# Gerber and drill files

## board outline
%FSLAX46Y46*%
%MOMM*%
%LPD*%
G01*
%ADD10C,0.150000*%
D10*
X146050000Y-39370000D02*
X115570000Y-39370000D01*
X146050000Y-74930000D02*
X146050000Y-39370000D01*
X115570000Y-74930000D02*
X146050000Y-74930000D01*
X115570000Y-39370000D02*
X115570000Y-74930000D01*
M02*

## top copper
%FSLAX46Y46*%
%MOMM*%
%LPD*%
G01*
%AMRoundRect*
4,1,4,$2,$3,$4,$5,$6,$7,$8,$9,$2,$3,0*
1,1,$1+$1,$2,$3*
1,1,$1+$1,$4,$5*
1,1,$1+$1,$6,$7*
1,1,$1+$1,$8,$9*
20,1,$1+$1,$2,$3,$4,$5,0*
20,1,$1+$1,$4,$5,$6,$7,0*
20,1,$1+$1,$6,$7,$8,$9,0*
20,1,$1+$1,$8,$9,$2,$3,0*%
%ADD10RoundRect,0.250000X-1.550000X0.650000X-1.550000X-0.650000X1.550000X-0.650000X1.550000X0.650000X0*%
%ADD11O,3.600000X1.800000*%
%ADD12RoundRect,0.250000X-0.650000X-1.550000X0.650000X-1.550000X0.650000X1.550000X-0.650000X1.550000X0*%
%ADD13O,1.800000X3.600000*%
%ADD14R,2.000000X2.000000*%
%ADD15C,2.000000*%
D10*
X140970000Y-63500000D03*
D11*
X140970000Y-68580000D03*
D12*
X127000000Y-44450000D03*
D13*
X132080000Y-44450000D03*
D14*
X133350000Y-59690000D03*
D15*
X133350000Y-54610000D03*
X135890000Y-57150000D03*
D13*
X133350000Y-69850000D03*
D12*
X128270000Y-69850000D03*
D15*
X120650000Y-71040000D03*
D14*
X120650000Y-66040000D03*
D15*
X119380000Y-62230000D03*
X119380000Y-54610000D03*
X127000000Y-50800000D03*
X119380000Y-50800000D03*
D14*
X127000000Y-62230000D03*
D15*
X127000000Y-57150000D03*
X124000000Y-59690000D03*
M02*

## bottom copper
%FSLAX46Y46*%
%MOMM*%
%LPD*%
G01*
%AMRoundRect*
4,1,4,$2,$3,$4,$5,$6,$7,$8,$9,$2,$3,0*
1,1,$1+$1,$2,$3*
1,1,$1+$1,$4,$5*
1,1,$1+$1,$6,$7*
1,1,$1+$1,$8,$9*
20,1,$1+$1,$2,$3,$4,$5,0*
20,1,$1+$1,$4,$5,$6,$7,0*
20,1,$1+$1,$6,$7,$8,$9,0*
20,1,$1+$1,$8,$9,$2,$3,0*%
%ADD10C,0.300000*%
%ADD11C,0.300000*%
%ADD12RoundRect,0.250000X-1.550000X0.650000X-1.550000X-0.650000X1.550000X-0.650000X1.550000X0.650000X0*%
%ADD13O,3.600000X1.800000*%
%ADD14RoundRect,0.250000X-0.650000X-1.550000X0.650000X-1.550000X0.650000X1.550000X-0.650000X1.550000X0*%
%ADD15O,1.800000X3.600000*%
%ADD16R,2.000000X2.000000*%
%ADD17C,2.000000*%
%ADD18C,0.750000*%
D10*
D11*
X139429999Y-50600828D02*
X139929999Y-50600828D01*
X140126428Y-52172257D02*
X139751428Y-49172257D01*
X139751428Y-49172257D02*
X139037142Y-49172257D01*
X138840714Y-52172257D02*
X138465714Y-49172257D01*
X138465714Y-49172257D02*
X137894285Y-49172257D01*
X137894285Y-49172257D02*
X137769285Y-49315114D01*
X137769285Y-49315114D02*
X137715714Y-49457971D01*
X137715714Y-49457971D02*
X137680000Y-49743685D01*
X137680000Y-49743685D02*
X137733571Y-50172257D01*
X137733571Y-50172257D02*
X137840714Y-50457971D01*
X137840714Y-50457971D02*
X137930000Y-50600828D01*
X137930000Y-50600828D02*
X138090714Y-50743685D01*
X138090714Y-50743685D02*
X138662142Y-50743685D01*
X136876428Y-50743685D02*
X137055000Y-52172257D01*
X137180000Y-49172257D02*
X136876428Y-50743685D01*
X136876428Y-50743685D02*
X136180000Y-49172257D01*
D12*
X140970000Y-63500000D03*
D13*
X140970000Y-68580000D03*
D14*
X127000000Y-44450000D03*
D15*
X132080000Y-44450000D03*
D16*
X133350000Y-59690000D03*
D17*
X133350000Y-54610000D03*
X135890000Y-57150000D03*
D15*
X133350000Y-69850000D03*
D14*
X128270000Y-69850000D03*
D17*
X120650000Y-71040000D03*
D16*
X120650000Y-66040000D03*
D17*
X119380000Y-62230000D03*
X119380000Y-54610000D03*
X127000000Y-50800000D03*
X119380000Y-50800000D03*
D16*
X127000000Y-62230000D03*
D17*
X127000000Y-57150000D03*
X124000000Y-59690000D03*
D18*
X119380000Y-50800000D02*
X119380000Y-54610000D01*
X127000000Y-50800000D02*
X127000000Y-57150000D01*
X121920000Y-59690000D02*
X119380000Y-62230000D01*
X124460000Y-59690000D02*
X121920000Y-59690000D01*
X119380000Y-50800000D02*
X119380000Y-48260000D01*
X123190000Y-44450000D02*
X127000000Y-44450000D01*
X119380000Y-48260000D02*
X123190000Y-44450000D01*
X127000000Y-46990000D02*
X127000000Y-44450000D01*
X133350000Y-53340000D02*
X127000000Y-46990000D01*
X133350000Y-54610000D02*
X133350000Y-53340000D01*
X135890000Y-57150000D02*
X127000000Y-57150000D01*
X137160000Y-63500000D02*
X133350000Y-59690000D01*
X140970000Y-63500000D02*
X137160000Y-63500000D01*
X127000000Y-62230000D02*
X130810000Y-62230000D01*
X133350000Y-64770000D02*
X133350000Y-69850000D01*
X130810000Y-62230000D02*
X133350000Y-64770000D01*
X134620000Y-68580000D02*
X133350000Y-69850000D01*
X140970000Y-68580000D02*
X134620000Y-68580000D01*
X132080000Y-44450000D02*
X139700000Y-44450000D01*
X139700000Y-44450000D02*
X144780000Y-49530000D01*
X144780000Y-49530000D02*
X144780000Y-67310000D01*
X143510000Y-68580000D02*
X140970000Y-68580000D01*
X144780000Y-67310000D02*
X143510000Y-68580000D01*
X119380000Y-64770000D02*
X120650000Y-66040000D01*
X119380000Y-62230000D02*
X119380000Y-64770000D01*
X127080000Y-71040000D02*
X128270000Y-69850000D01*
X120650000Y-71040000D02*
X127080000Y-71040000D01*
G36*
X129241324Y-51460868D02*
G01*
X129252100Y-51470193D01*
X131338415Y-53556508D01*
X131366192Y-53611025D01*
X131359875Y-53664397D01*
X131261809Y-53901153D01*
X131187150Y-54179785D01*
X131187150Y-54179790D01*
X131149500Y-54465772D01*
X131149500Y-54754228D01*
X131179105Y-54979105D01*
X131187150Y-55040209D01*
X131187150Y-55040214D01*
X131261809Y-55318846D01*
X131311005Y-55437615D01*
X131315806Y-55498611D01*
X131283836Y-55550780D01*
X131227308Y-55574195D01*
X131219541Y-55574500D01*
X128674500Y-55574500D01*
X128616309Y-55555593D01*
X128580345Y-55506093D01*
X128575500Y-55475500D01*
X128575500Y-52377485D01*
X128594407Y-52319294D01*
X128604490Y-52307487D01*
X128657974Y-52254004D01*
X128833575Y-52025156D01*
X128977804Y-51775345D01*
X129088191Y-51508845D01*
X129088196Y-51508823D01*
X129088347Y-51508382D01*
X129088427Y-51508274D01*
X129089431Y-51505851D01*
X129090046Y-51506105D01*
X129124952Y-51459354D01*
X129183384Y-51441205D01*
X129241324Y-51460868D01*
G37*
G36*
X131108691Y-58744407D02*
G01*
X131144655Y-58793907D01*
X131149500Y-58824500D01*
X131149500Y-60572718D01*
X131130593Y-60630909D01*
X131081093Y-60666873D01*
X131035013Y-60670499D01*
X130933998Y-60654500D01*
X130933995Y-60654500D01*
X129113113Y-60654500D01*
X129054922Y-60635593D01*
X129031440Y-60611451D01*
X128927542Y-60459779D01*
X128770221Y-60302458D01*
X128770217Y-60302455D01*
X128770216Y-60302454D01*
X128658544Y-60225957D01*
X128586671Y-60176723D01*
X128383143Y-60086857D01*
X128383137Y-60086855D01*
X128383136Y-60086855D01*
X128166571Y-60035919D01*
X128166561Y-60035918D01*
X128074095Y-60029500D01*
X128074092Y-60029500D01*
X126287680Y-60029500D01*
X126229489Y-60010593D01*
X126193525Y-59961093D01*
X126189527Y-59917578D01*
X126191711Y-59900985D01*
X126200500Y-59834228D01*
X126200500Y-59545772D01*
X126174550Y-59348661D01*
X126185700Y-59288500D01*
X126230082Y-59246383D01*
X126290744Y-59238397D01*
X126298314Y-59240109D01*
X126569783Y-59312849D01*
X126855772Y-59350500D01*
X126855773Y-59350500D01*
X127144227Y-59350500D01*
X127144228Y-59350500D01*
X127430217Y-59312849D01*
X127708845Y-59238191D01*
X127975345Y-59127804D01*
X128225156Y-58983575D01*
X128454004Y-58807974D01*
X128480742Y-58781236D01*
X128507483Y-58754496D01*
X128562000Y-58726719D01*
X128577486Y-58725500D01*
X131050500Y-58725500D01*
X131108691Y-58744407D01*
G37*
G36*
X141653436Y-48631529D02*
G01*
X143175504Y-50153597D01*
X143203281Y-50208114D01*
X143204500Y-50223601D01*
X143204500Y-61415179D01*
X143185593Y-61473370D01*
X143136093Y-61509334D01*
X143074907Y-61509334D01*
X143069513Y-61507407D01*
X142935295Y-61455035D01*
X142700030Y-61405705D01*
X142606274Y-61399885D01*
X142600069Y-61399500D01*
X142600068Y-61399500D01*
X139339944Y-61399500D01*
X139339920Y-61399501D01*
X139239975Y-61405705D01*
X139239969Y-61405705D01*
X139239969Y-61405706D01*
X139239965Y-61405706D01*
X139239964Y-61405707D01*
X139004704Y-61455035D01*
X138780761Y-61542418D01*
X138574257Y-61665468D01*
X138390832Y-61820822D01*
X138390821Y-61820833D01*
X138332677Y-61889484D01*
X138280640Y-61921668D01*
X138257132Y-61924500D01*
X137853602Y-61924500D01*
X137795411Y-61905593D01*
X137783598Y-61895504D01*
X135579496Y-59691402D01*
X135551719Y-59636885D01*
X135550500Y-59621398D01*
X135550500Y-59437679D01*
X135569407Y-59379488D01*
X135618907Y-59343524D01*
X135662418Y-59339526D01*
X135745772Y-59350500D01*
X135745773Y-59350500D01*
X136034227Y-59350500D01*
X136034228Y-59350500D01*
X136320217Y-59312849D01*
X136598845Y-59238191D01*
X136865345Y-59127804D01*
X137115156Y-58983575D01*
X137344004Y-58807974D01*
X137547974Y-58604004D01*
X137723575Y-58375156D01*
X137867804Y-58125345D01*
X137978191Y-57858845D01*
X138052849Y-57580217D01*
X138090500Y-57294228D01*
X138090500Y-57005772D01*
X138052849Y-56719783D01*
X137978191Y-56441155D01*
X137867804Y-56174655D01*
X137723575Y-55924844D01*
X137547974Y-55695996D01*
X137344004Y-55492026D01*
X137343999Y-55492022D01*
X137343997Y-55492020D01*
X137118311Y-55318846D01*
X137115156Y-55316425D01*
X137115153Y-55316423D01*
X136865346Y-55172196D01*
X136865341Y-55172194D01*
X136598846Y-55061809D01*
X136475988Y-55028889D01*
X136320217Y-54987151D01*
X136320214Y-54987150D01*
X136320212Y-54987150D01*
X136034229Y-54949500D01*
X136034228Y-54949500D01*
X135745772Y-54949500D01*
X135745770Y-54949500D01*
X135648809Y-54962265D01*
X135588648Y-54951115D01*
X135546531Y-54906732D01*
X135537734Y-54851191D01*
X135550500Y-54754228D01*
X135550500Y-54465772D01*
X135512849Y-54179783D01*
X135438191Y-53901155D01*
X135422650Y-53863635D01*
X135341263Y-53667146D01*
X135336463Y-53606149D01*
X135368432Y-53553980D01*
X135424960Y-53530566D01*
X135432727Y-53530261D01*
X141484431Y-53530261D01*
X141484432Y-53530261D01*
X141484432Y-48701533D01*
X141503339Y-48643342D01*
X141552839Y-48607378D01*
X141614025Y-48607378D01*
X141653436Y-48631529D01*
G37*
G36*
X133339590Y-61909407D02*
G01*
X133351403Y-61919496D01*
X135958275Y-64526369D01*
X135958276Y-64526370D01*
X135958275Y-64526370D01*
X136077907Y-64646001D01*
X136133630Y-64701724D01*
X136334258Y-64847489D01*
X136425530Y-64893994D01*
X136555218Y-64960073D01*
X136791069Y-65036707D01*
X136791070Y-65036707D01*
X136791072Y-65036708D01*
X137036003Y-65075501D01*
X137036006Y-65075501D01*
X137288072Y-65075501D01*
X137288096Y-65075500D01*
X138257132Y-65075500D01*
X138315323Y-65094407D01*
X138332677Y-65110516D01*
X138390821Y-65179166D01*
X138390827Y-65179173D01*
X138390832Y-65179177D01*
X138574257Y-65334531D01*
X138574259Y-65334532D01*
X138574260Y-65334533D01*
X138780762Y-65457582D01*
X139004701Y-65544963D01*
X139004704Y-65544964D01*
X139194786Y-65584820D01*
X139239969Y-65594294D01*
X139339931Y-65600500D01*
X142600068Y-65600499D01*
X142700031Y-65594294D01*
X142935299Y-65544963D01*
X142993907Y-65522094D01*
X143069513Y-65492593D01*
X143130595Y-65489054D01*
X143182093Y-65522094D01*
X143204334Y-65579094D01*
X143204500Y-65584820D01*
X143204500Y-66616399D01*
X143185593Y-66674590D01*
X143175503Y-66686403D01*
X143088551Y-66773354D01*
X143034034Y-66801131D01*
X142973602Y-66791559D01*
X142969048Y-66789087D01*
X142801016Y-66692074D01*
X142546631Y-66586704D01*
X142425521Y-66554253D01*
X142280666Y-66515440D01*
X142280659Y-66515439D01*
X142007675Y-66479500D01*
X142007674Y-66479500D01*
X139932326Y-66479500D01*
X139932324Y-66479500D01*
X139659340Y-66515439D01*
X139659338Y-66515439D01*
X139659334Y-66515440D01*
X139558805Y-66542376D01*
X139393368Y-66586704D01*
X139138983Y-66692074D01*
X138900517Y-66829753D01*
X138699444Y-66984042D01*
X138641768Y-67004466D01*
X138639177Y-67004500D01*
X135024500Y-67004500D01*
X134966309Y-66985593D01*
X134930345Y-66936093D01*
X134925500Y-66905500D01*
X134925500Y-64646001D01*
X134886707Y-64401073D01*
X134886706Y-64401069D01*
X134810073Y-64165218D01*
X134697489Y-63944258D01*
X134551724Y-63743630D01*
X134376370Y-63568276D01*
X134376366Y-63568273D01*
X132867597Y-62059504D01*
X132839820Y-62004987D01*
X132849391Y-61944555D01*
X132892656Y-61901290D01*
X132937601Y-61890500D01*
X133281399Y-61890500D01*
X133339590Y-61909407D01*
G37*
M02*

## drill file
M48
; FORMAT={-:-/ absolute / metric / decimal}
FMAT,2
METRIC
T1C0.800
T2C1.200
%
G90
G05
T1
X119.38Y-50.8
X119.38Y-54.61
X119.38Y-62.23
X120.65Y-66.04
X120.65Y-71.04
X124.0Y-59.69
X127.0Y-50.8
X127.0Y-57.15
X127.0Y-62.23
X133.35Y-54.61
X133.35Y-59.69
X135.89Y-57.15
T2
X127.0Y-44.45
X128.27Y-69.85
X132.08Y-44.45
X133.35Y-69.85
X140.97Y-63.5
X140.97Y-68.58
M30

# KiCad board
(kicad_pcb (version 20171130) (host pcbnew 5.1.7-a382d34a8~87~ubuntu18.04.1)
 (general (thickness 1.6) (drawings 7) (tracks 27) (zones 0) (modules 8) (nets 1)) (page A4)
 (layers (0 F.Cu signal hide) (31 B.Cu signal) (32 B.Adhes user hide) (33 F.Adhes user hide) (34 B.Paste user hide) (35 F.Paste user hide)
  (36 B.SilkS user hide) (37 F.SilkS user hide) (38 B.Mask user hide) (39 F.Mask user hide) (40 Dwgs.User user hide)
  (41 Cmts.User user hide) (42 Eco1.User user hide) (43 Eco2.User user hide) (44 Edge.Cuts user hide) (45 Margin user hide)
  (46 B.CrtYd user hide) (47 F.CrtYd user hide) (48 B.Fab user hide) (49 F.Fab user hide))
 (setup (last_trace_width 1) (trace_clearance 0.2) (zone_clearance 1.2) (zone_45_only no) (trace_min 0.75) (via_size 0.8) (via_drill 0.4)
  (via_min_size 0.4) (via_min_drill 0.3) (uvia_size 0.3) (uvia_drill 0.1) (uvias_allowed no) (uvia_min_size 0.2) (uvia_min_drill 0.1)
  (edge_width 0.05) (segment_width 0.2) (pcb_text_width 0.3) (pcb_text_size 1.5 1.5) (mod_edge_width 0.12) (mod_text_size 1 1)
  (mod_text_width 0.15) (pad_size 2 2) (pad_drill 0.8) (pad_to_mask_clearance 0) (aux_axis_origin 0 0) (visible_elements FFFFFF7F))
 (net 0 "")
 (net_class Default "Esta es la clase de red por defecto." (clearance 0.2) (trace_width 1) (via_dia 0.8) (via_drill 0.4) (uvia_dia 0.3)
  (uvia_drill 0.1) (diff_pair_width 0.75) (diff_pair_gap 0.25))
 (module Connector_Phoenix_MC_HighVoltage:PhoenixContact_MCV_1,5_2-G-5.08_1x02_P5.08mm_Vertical (layer F.Cu) (at 140.97 63.5 270)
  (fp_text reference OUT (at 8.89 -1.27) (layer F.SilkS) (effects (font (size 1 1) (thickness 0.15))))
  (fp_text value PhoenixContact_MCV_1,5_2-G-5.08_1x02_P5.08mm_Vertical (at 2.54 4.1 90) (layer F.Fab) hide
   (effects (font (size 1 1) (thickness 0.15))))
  (pad 1 thru_hole roundrect (at 0 0 270) (size 1.8 3.6) (drill 1.2) (layers *.Cu *.Mask) (roundrect_rratio 0.1388888888888889))
  (pad 2 thru_hole oval (at 5.08 0 270) (size 1.8 3.6) (drill 1.2) (layers *.Cu *.Mask)))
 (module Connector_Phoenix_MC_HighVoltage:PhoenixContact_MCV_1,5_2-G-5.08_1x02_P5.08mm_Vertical (layer F.Cu) (at 127 44.45)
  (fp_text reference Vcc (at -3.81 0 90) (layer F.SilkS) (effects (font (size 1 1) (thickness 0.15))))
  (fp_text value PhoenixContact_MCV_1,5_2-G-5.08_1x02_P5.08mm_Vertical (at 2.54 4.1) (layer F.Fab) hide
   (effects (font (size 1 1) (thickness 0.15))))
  (pad 1 thru_hole roundrect (at 0 0) (size 1.8 3.6) (drill 1.2) (layers *.Cu *.Mask) (roundrect_rratio 0.1388888888888889))
  (pad 2 thru_hole oval (at 5.08 0) (size 1.8 3.6) (drill 1.2) (layers *.Cu *.Mask)))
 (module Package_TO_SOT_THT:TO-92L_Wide (layer B.Cu) (at 133.35 59.69 90)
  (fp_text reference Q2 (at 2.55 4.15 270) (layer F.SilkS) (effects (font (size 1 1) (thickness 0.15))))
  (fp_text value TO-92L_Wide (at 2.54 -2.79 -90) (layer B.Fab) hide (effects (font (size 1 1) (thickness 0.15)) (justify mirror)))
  (pad 1 thru_hole rect (at 0 0 90) (size 2 2) (drill 0.8) (layers *.Cu *.Mask))
  (pad 3 thru_hole circle (at 5.08 0 90) (size 2 2) (drill 0.8) (layers *.Cu *.Mask))
  (pad 2 thru_hole circle (at 2.54 2.54 90) (size 2 2) (drill 0.8) (layers *.Cu *.Mask)))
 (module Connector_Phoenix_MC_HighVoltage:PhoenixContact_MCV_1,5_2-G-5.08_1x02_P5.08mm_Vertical (layer B.Cu) (at 128.27 69.85)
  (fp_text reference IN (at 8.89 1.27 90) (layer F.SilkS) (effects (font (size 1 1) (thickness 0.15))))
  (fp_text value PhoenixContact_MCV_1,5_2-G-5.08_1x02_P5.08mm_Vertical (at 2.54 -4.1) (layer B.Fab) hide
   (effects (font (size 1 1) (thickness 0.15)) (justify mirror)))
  (pad 2 thru_hole oval (at 5.08 0) (size 1.8 3.6) (drill 1.2) (layers *.Cu *.Mask))
  (pad 1 thru_hole roundrect (at 0 0) (size 1.8 3.6) (drill 1.2) (layers *.Cu *.Mask) (roundrect_rratio 0.1388888888888889)))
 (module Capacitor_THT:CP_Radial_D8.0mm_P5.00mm (layer F.Cu) (at 120.65 66.04 270)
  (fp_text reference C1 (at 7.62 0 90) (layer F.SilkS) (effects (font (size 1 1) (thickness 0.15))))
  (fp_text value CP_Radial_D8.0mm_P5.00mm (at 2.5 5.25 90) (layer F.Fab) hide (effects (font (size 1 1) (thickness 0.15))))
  (pad 2 thru_hole circle (at 5 0 270) (size 2 2) (drill 0.8) (layers *.Cu *.Mask))
  (pad 1 thru_hole rect (at 0 0 270) (size 2 2) (drill 0.8) (layers *.Cu *.Mask)))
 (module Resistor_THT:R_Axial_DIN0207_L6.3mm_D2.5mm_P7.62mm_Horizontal (layer F.Cu) (at 119.38 62.23 90)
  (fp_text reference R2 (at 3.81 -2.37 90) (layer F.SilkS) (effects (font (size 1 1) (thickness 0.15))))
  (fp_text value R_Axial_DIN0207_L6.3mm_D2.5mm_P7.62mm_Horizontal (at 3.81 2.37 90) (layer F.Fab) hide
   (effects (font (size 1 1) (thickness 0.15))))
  (pad 1 thru_hole circle (at 0 0 90) (size 2 2) (drill 0.8) (layers *.Cu *.Mask))
  (pad 2 thru_hole circle (at 7.62 0 90) (size 2 2) (drill 0.8) (layers *.Cu *.Mask)))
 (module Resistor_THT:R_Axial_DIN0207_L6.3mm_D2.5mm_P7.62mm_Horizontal (layer F.Cu) (at 119.38 50.8)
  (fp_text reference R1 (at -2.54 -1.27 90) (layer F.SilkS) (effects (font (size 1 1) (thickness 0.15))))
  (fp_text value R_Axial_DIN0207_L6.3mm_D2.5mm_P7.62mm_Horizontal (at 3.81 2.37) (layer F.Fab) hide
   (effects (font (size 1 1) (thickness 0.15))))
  (pad 2 thru_hole circle (at 7.62 0) (size 2 2) (drill 0.8) (layers *.Cu *.Mask))
  (pad 1 thru_hole circle (at 0 0) (size 2 2) (drill 0.8) (layers *.Cu *.Mask)))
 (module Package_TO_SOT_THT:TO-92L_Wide (layer F.Cu) (at 127 62.23 90)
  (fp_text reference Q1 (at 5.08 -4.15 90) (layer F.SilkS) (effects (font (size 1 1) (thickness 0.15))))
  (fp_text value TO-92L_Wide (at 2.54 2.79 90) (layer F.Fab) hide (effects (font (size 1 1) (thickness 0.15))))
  (pad 1 thru_hole rect (at 0 0 90) (size 2 2) (drill 0.8) (layers *.Cu *.Mask))
  (pad 3 thru_hole circle (at 5.08 0 90) (size 2 2) (drill 0.8) (layers *.Cu *.Mask))
  (pad 2 thru_hole circle (at 2.54 -3 90) (size 2 2) (drill 0.8) (layers *.Cu *.Mask)))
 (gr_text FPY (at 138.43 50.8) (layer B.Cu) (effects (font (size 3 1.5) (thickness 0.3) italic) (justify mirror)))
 (gr_line (start 146.05 39.37) (end 115.57 39.37) (layer Edge.Cuts) (width 0.15))
 (gr_line (start 146.05 74.93) (end 146.05 39.37) (layer Edge.Cuts) (width 0.15))
 (gr_line (start 115.57 74.93) (end 146.05 74.93) (layer Edge.Cuts) (width 0.15))
 (gr_line (start 115.57 39.37) (end 115.57 74.93) (layer Edge.Cuts) (width 0.15))
 (segment (start 119.38 50.8) (end 119.38 54.61) (width 0.75) (layer B.Cu) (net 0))
 (segment (start 127 50.8) (end 127 57.15) (width 0.75) (layer B.Cu) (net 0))
 (segment (start 121.92 59.69) (end 119.38 62.23) (width 0.75) (layer B.Cu) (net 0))
 (segment (start 124.46 59.69) (end 121.92 59.69) (width 0.75) (layer B.Cu) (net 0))
 (segment (start 119.38 50.8) (end 119.38 48.26) (width 0.75) (layer B.Cu) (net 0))
 (segment (start 123.19 44.45) (end 127 44.45) (width 0.75) (layer B.Cu) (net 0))
 (segment (start 119.38 48.26) (end 123.19 44.45) (width 0.75) (layer B.Cu) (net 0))
 (segment (start 127 46.99) (end 127 44.45) (width 0.75) (layer B.Cu) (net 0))
 (segment (start 133.35 53.34) (end 127 46.99) (width 0.75) (layer B.Cu) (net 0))
 (segment (start 133.35 54.61) (end 133.35 53.34) (width 0.75) (layer B.Cu) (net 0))
 (segment (start 135.89 57.15) (end 127 57.15) (width 0.75) (layer B.Cu) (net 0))
 (segment (start 137.16 63.5) (end 133.35 59.69) (width 0.75) (layer B.Cu) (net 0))
 (segment (start 140.97 63.5) (end 137.16 63.5) (width 0.75) (layer B.Cu) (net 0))
 (segment (start 127 62.23) (end 130.81 62.23) (width 0.75) (layer B.Cu) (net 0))
 (segment (start 133.35 64.77) (end 133.35 69.85) (width 0.75) (layer B.Cu) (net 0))
 (segment (start 130.81 62.23) (end 133.35 64.77) (width 0.75) (layer B.Cu) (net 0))
 (segment (start 134.62 68.58) (end 133.35 69.85) (width 0.75) (layer B.Cu) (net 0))
 (segment (start 140.97 68.58) (end 134.62 68.58) (width 0.75) (layer B.Cu) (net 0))
 (segment (start 132.08 44.45) (end 139.7 44.45) (width 0.75) (layer B.Cu) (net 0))
 (segment (start 139.7 44.45) (end 144.78 49.53) (width 0.75) (layer B.Cu) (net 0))
 (segment (start 144.78 49.53) (end 144.78 67.31) (width 0.75) (layer B.Cu) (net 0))
 (segment (start 143.51 68.58) (end 140.97 68.58) (width 0.75) (layer B.Cu) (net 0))
 (segment (start 144.78 67.31) (end 143.51 68.58) (width 0.75) (layer B.Cu) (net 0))
 (segment (start 119.38 64.77) (end 120.65 66.04) (width 0.75) (layer B.Cu) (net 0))
 (segment (start 119.38 62.23) (end 119.38 64.77) (width 0.75) (layer B.Cu) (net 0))
 (segment (start 127.08 71.04) (end 128.27 69.85) (width 0.75) (layer B.Cu) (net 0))
 (segment (start 120.65 71.04) (end 127.08 71.04) (width 0.75) (layer B.Cu) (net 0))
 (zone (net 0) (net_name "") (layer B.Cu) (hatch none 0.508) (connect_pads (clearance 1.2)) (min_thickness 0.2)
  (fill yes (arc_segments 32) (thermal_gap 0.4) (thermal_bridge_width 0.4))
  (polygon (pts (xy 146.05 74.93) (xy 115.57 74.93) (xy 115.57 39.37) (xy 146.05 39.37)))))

